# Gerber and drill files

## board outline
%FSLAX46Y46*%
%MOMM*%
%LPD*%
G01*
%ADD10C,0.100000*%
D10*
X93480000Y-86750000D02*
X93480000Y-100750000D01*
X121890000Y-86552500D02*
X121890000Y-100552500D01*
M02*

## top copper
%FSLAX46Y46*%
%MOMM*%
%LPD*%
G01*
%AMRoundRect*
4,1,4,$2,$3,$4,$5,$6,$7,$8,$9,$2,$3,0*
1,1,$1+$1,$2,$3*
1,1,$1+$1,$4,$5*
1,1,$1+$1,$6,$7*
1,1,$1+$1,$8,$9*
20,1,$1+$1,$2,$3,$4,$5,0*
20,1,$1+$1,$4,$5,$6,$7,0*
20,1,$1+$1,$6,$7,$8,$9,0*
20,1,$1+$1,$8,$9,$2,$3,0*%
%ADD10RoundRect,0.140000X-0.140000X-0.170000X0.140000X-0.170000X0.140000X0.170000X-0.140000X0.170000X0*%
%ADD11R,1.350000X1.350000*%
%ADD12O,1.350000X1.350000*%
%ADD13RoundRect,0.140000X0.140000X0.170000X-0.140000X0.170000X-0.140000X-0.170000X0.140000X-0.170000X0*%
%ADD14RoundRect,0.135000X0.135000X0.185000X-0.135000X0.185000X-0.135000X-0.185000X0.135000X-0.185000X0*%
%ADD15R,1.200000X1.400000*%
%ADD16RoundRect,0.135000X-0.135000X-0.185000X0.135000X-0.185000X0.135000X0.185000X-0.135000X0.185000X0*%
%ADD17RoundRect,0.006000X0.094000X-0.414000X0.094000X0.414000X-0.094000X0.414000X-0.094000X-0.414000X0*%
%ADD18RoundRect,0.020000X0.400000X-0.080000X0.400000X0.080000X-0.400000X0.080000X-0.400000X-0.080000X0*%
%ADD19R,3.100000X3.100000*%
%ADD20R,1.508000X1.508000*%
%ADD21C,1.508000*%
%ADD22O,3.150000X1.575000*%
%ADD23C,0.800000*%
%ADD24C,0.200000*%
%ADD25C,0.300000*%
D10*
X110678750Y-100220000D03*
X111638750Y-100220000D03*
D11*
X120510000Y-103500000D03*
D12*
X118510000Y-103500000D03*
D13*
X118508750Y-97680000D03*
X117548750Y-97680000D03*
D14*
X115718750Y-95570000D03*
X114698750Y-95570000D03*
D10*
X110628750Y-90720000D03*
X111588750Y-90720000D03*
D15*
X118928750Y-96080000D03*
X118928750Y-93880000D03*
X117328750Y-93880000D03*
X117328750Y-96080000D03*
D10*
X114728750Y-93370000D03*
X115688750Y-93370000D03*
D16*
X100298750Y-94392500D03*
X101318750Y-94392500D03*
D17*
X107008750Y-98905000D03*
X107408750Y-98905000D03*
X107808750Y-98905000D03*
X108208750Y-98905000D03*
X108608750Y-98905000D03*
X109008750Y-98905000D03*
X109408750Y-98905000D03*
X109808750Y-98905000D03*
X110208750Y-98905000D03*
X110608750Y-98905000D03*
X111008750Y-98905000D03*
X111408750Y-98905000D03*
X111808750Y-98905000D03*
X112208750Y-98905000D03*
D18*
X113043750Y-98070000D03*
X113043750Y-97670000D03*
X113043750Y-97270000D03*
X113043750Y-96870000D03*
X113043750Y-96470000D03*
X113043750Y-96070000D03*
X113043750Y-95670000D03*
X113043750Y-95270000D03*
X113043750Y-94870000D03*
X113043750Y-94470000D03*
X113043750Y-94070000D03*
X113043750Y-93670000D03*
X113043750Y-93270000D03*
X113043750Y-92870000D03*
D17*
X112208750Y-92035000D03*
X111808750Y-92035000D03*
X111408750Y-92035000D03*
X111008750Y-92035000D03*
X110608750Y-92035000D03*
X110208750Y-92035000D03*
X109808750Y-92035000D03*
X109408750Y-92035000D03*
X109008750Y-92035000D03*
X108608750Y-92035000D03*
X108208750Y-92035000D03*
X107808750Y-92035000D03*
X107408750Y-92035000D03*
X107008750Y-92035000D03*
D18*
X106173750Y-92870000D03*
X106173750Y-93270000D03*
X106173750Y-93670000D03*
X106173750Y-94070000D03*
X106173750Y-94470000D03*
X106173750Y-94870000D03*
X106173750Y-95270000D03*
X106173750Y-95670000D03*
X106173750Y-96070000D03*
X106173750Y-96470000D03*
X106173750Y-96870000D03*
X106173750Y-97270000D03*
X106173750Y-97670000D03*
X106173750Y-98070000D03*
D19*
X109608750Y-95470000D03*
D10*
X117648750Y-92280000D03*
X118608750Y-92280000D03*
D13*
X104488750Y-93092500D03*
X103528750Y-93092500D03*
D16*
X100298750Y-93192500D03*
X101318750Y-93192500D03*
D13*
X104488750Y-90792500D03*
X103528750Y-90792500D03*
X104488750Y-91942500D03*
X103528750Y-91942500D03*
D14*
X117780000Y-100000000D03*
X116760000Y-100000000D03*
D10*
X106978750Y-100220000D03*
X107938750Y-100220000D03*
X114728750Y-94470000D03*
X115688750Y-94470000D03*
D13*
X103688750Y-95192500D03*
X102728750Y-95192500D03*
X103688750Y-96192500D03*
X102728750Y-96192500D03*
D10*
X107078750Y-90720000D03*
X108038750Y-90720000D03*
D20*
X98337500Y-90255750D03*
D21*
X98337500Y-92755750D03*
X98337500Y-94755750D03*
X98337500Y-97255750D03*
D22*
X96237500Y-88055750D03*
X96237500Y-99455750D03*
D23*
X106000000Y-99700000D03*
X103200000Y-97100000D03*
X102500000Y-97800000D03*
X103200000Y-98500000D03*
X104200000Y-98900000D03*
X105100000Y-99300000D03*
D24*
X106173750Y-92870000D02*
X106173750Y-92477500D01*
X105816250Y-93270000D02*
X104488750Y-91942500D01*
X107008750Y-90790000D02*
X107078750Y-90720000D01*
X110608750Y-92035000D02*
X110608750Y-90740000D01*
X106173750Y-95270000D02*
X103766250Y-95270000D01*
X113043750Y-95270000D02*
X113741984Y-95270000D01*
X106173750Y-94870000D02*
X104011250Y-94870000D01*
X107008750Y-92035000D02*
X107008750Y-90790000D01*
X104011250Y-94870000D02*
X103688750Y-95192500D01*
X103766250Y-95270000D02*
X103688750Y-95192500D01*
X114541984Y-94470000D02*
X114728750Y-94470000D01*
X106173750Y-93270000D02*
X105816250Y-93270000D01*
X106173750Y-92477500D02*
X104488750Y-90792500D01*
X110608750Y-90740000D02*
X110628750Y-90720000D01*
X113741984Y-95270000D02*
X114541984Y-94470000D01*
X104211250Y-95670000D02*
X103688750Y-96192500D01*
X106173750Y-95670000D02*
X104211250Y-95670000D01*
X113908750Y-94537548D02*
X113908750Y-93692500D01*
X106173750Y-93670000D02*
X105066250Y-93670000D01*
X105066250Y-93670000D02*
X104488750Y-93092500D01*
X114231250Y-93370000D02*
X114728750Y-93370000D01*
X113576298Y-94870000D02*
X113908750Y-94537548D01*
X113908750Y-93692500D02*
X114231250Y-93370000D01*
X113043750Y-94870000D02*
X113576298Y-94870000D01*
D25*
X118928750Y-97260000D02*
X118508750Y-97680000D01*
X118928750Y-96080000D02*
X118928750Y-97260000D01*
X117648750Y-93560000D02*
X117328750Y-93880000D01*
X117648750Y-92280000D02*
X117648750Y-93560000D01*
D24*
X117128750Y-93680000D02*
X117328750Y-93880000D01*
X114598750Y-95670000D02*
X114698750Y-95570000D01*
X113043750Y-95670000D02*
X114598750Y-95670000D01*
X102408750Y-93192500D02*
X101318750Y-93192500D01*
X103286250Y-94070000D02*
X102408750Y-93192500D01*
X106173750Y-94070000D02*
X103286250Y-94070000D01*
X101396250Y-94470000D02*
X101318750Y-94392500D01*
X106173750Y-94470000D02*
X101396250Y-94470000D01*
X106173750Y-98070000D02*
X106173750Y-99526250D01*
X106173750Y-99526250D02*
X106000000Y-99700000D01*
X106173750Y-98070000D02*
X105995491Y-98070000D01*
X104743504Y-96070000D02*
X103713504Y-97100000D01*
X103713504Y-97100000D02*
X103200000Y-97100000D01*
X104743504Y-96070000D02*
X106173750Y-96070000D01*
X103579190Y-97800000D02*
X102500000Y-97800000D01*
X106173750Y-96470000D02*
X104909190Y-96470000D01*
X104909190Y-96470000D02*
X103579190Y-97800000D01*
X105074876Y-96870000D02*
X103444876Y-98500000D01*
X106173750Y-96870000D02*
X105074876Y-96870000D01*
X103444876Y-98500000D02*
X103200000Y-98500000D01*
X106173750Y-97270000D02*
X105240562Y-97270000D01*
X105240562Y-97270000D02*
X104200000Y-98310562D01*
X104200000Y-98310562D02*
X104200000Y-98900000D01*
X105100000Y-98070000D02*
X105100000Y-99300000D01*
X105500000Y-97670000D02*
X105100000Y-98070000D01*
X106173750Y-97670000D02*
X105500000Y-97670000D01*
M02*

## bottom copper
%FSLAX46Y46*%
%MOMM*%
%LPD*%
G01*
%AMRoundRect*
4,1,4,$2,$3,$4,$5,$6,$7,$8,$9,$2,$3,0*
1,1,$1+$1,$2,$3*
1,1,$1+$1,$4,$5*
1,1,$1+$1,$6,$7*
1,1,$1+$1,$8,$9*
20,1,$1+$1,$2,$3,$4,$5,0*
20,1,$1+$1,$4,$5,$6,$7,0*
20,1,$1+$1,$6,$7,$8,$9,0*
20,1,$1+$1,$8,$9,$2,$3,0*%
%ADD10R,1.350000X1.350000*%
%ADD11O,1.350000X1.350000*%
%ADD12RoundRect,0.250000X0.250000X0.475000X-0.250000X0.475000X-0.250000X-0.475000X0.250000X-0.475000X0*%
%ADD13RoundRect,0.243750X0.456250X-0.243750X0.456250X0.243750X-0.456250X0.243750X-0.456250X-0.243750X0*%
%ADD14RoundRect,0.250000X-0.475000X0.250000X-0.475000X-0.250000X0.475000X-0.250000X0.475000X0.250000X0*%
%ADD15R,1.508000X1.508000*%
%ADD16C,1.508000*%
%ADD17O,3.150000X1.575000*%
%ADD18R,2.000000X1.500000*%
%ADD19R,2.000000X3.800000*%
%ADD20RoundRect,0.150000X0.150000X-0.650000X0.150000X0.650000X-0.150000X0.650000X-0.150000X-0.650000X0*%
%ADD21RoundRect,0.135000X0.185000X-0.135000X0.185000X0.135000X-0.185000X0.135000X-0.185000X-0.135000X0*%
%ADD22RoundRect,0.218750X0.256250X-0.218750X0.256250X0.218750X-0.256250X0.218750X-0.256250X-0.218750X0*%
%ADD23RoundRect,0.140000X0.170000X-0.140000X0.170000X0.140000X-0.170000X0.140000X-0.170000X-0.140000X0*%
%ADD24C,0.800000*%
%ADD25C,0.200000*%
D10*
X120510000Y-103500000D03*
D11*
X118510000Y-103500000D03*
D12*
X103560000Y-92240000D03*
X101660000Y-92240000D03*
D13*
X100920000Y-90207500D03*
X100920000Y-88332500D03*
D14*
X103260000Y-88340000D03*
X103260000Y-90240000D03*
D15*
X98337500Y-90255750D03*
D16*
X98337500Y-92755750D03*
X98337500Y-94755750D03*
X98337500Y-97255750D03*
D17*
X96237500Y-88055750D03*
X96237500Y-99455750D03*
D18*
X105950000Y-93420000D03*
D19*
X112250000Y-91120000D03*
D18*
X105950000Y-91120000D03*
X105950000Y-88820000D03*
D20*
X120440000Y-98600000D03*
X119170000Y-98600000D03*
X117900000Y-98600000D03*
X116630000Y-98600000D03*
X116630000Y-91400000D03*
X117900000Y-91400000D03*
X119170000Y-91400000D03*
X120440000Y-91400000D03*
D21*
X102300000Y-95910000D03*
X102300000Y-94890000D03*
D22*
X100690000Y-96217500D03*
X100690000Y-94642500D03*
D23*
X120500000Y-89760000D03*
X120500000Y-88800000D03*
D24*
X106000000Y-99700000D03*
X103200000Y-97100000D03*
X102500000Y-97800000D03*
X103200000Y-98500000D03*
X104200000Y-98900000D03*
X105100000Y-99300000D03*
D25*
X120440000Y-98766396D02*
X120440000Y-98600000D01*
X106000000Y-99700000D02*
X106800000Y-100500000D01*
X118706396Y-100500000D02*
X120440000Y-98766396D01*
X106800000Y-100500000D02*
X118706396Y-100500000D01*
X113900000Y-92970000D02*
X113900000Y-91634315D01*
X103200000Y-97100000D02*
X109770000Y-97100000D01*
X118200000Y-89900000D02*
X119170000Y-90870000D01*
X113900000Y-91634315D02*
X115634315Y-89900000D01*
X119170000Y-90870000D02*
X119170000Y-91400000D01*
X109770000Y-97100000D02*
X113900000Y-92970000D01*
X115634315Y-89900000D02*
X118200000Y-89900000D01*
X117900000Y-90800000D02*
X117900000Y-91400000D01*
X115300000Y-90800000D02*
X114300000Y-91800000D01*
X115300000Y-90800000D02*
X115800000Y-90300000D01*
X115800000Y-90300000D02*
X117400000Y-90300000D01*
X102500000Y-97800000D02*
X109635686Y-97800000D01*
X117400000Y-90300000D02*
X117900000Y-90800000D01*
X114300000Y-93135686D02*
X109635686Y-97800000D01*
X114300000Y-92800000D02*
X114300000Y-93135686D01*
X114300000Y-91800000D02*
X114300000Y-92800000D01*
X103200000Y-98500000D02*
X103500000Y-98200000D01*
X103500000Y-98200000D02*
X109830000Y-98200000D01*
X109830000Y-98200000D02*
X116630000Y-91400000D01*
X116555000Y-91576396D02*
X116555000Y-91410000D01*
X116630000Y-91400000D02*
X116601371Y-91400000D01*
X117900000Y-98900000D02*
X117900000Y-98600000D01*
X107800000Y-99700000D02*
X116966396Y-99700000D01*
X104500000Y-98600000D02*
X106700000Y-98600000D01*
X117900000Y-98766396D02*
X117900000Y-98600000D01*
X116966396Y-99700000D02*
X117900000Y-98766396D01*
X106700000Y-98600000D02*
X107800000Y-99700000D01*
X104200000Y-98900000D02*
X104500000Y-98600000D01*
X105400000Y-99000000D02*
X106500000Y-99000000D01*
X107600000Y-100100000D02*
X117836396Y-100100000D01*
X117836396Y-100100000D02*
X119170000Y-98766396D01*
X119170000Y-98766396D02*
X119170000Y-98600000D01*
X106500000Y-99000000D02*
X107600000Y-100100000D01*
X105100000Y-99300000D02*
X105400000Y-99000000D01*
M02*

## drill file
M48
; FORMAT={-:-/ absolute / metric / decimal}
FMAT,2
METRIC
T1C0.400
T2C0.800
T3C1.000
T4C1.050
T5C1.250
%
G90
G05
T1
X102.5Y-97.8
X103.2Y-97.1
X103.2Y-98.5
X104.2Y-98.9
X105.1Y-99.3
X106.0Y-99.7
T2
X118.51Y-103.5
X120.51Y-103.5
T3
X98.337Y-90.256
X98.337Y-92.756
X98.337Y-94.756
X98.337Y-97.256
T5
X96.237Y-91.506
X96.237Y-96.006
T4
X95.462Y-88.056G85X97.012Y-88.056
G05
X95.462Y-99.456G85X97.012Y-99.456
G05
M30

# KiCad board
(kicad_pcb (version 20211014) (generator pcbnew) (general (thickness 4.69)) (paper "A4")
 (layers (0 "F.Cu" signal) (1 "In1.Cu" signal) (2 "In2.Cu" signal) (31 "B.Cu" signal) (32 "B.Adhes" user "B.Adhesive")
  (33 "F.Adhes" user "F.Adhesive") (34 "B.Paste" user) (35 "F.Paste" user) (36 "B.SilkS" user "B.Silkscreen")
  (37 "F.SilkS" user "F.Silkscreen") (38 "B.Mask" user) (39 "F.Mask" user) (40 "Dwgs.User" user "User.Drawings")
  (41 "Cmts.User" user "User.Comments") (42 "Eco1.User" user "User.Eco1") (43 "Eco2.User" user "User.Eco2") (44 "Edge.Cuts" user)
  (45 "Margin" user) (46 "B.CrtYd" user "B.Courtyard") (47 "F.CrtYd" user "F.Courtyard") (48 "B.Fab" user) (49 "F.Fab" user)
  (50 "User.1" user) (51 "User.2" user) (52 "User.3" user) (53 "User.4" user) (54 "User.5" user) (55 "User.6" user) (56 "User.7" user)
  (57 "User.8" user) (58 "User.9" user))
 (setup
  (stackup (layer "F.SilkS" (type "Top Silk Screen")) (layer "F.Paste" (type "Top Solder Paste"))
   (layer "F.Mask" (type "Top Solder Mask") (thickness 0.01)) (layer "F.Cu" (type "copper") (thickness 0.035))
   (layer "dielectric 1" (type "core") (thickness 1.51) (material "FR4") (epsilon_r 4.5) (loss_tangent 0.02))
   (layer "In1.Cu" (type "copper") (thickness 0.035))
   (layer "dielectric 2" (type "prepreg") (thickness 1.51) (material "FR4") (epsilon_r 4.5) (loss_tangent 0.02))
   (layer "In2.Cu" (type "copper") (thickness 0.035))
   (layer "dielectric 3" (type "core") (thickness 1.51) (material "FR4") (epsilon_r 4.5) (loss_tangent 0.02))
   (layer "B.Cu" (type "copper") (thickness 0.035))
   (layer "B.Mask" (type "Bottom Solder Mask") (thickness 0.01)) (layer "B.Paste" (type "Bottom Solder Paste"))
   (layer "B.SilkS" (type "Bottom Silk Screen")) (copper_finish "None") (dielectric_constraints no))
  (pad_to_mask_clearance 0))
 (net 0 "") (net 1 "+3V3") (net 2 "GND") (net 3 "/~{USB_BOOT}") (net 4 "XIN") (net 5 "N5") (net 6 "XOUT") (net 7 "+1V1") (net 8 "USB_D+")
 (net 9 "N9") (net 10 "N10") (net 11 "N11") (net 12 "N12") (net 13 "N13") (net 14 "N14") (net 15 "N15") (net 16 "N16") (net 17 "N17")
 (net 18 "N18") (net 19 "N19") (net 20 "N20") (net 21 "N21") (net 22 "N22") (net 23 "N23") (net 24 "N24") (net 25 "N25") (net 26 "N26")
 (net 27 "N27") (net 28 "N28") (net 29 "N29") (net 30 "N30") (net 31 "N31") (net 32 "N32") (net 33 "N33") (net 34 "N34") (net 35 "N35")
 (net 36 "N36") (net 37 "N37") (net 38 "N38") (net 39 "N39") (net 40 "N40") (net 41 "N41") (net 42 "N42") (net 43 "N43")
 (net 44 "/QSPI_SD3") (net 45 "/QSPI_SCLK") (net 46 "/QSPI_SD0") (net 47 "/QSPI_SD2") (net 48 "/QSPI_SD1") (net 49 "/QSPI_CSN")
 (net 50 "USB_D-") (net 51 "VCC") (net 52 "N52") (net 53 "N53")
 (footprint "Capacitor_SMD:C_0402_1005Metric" (layer "F.Cu") (at 111.15875 100.22)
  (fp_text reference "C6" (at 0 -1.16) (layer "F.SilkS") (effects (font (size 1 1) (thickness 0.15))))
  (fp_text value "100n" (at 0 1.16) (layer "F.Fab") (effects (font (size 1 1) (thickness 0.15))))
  (pad "1" smd roundrect (at -0.48 0) (size 0.56 0.62) (layers "F.Cu" "F.Paste" "F.Mask") (roundrect_rratio 0.25) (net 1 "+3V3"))
  (pad "2" smd roundrect (at 0.48 0) (size 0.56 0.62) (layers "F.Cu" "F.Paste" "F.Mask") (roundrect_rratio 0.25) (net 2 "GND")))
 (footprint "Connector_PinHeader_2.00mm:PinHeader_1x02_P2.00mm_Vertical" (layer "F.Cu") (at 120.51 103.5 -90)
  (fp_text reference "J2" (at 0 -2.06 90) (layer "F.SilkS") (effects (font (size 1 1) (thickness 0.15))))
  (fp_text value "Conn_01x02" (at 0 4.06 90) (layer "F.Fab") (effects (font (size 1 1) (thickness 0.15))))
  (pad "1" thru_hole rect (at 0 0 270) (size 1.35 1.35) (drill 0.8) (layers *.Cu *.Mask) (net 2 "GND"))
  (pad "2" thru_hole oval (at 0 2 270) (size 1.35 1.35) (drill 0.8) (layers *.Cu *.Mask) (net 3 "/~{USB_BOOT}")))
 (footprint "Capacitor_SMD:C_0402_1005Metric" (layer "F.Cu") (at 118.02875 97.68 180)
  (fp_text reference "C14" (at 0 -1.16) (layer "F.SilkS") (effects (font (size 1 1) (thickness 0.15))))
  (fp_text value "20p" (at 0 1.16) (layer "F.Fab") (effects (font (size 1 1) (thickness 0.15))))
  (pad "1" smd roundrect (at -0.48 0 180) (size 0.56 0.62) (layers "F.Cu" "F.Paste" "F.Mask") (roundrect_rratio 0.25) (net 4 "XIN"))
  (pad "2" smd roundrect (at 0.48 0 180) (size 0.56 0.62) (layers "F.Cu" "F.Paste" "F.Mask") (roundrect_rratio 0.25) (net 2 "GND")))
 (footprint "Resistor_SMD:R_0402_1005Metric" (layer "F.Cu") (at 115.20875 95.57 180)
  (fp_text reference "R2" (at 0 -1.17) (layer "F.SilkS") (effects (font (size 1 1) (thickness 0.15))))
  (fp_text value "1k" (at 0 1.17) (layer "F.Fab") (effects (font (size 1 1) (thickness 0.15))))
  (pad "1" smd roundrect (at -0.51 0 180) (size 0.54 0.64) (layers "F.Cu" "F.Paste" "F.Mask") (roundrect_rratio 0.25) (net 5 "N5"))
  (pad "2" smd roundrect (at 0.51 0 180) (size 0.54 0.64) (layers "F.Cu" "F.Paste" "F.Mask") (roundrect_rratio 0.25) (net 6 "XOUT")))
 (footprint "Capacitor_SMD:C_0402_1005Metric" (layer "F.Cu") (at 111.10875 90.72)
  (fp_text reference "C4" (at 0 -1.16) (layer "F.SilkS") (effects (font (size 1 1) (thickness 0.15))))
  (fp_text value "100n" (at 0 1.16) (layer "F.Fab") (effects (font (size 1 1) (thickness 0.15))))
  (pad "1" smd roundrect (at -0.48 0) (size 0.56 0.62) (layers "F.Cu" "F.Paste" "F.Mask") (roundrect_rratio 0.25) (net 1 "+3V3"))
  (pad "2" smd roundrect (at 0.48 0) (size 0.56 0.62) (layers "F.Cu" "F.Paste" "F.Mask") (roundrect_rratio 0.25) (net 2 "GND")))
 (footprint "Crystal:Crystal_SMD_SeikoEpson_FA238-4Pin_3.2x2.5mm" (layer "F.Cu") (at 118.12875 94.98 90)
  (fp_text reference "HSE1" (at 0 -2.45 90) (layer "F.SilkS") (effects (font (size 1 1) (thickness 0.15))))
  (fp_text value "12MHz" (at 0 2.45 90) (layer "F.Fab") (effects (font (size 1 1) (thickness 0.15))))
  (pad "1" smd rect (at -1.1 0.8 90) (size 1.4 1.2) (layers "F.Cu" "F.Paste" "F.Mask") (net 4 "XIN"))
  (pad "2" smd rect (at 1.1 0.8 90) (size 1.4 1.2) (layers "F.Cu" "F.Paste" "F.Mask") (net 2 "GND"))
  (pad "3" smd rect (at 1.1 -0.8 90) (size 1.4 1.2) (layers "F.Cu" "F.Paste" "F.Mask") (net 5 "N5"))
  (pad "4" smd rect (at -1.1 -0.8 90) (size 1.4 1.2) (layers "F.Cu" "F.Paste" "F.Mask") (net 2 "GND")))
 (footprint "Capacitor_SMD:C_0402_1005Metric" (layer "F.Cu") (at 115.20875 93.37)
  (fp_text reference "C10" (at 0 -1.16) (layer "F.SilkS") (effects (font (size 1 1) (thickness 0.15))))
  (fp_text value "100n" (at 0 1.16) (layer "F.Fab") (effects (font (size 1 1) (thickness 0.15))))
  (pad "1" smd roundrect (at -0.48 0) (size 0.56 0.62) (layers "F.Cu" "F.Paste" "F.Mask") (roundrect_rratio 0.25) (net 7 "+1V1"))
  (pad "2" smd roundrect (at 0.48 0) (size 0.56 0.62) (layers "F.Cu" "F.Paste" "F.Mask") (roundrect_rratio 0.25) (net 2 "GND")))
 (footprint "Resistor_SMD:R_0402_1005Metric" (layer "F.Cu") (at 100.80875 94.3925)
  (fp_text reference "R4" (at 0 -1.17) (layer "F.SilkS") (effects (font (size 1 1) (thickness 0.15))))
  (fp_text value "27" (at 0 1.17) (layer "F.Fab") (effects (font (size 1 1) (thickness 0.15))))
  (pad "1" smd roundrect (at -0.51 0) (size 0.54 0.64) (layers "F.Cu" "F.Paste" "F.Mask") (roundrect_rratio 0.25) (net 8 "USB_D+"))
  (pad "2" smd roundrect (at 0.51 0) (size 0.54 0.64) (layers "F.Cu" "F.Paste" "F.Mask") (roundrect_rratio 0.25) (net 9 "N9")))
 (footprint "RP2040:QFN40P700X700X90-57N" (layer "F.Cu") (at 109.60875 95.47 90)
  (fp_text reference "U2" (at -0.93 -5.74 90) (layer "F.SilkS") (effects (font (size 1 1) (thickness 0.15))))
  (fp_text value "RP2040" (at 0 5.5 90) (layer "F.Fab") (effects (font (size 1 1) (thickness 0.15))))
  (pad "1" smd roundrect locked (at -3.435 -2.6 90) (size 0.84 0.2) (layers "F.Cu" "F.Paste" "F.Mask") (roundrect_rratio 0.03)
   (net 1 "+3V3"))
  (pad "2" smd roundrect locked (at -3.435 -2.2 90) (size 0.84 0.2) (layers "F.Cu" "F.Paste" "F.Mask") (roundrect_rratio 0.03)
   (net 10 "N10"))
  (pad "3" smd roundrect locked (at -3.435 -1.8 90) (size 0.84 0.2) (layers "F.Cu" "F.Paste" "F.Mask") (roundrect_rratio 0.03)
   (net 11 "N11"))
  (pad "4" smd roundrect locked (at -3.435 -1.4 90) (size 0.84 0.2) (layers "F.Cu" "F.Paste" "F.Mask") (roundrect_rratio 0.03)
   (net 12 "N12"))
  (pad "5" smd roundrect locked (at -3.435 -1 90) (size 0.84 0.2) (layers "F.Cu" "F.Paste" "F.Mask") (roundrect_rratio 0.03) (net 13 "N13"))
  (pad "6" smd roundrect locked (at -3.435 -0.6 90) (size 0.84 0.2) (layers "F.Cu" "F.Paste" "F.Mask") (roundrect_rratio 0.03)
   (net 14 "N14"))
  (pad "7" smd roundrect locked (at -3.435 -0.2 90) (size 0.84 0.2) (layers "F.Cu" "F.Paste" "F.Mask") (roundrect_rratio 0.03)
   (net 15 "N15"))
  (pad "8" smd roundrect locked (at -3.435 0.2 90) (size 0.84 0.2) (layers "F.Cu" "F.Paste" "F.Mask") (roundrect_rratio 0.03) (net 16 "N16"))
  (pad "9" smd roundrect locked (at -3.435 0.6 90) (size 0.84 0.2) (layers "F.Cu" "F.Paste" "F.Mask") (roundrect_rratio 0.03) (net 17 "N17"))
  (pad "10" smd roundrect locked (at -3.435 1 90) (size 0.84 0.2) (layers "F.Cu" "F.Paste" "F.Mask") (roundrect_rratio 0.03) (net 1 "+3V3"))
  (pad "11" smd roundrect locked (at -3.435 1.4 90) (size 0.84 0.2) (layers "F.Cu" "F.Paste" "F.Mask") (roundrect_rratio 0.03)
   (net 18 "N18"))
  (pad "12" smd roundrect locked (at -3.435 1.8 90) (size 0.84 0.2) (layers "F.Cu" "F.Paste" "F.Mask") (roundrect_rratio 0.03)
   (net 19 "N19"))
  (pad "13" smd roundrect locked (at -3.435 2.2 90) (size 0.84 0.2) (layers "F.Cu" "F.Paste" "F.Mask") (roundrect_rratio 0.03)
   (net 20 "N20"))
  (pad "14" smd roundrect locked (at -3.435 2.6 90) (size 0.84 0.2) (layers "F.Cu" "F.Paste" "F.Mask") (roundrect_rratio 0.03)
   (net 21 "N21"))
  (pad "15" smd roundrect locked (at -2.6 3.435 90) (size 0.2 0.84) (layers "F.Cu" "F.Paste" "F.Mask") (roundrect_rratio 0.1) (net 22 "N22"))
  (pad "16" smd roundrect locked (at -2.2 3.435 90) (size 0.2 0.84) (layers "F.Cu" "F.Paste" "F.Mask") (roundrect_rratio 0.1) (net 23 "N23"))
  (pad "17" smd roundrect locked (at -1.8 3.435 90) (size 0.2 0.84) (layers "F.Cu" "F.Paste" "F.Mask") (roundrect_rratio 0.1) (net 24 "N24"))
  (pad "18" smd roundrect locked (at -1.4 3.435 90) (size 0.2 0.84) (layers "F.Cu" "F.Paste" "F.Mask") (roundrect_rratio 0.1) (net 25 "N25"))
  (pad "19" smd roundrect locked (at -1 3.435 90) (size 0.2 0.84) (layers "F.Cu" "F.Paste" "F.Mask") (roundrect_rratio 0.1) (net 2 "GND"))
  (pad "20" smd roundrect locked (at -0.6 3.435 90) (size 0.2 0.84) (layers "F.Cu" "F.Paste" "F.Mask") (roundrect_rratio 0.1) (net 4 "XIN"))
  (pad "21" smd roundrect locked (at -0.2 3.435 90) (size 0.2 0.84) (layers "F.Cu" "F.Paste" "F.Mask") (roundrect_rratio 0.1) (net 6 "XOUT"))
  (pad "22" smd roundrect locked (at 0.2 3.435 90) (size 0.2 0.84) (layers "F.Cu" "F.Paste" "F.Mask") (roundrect_rratio 0.1) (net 1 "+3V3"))
  (pad "23" smd roundrect locked (at 0.6 3.435 90) (size 0.2 0.84) (layers "F.Cu" "F.Paste" "F.Mask") (roundrect_rratio 0.1) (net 7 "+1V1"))
  (pad "24" smd roundrect locked (at 1 3.435 90) (size 0.2 0.84) (layers "F.Cu" "F.Paste" "F.Mask") (roundrect_rratio 0.1) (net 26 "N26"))
  (pad "25" smd roundrect locked (at 1.4 3.435 90) (size 0.2 0.84) (layers "F.Cu" "F.Paste" "F.Mask") (roundrect_rratio 0.1) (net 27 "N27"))
  (pad "26" smd roundrect locked (at 1.8 3.435 90) (size 0.2 0.84) (layers "F.Cu" "F.Paste" "F.Mask") (roundrect_rratio 0.1) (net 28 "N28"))
  (pad "27" smd roundrect locked (at 2.2 3.435 90) (size 0.2 0.84) (layers "F.Cu" "F.Paste" "F.Mask") (roundrect_rratio 0.1) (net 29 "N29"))
  (pad "28" smd roundrect locked (at 2.6 3.435 90) (size 0.2 0.84) (layers "F.Cu" "F.Paste" "F.Mask") (roundrect_rratio 0.1) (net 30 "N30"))
  (pad "29" smd roundrect locked (at 3.435 2.6 90) (size 0.84 0.2) (layers "F.Cu" "F.Paste" "F.Mask") (roundrect_rratio 0.03) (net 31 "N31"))
  (pad "30" smd roundrect locked (at 3.435 2.2 90) (size 0.84 0.2) (layers "F.Cu" "F.Paste" "F.Mask") (roundrect_rratio 0.03) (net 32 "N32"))
  (pad "31" smd roundrect locked (at 3.435 1.8 90) (size 0.84 0.2) (layers "F.Cu" "F.Paste" "F.Mask") (roundrect_rratio 0.03) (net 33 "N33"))
  (pad "32" smd roundrect locked (at 3.435 1.4 90) (size 0.84 0.2) (layers "F.Cu" "F.Paste" "F.Mask") (roundrect_rratio 0.03) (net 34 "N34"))
  (pad "33" smd roundrect locked (at 3.435 1 90) (size 0.84 0.2) (layers "F.Cu" "F.Paste" "F.Mask") (roundrect_rratio 0.03) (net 1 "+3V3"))
  (pad "34" smd roundrect locked (at 3.435 0.6 90) (size 0.84 0.2) (layers "F.Cu" "F.Paste" "F.Mask") (roundrect_rratio 0.03) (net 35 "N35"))
  (pad "35" smd roundrect locked (at 3.435 0.2 90) (size 0.84 0.2) (layers "F.Cu" "F.Paste" "F.Mask") (roundrect_rratio 0.03) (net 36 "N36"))
  (pad "36" smd roundrect locked (at 3.435 -0.2 90) (size 0.84 0.2) (layers "F.Cu" "F.Paste" "F.Mask") (roundrect_rratio 0.03)
   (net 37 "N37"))
  (pad "37" smd roundrect locked (at 3.435 -0.6 90) (size 0.84 0.2) (layers "F.Cu" "F.Paste" "F.Mask") (roundrect_rratio 0.03)
   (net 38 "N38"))
  (pad "38" smd roundrect locked (at 3.435 -1 90) (size 0.84 0.2) (layers "F.Cu" "F.Paste" "F.Mask") (roundrect_rratio 0.03) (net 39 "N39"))
  (pad "39" smd roundrect locked (at 3.435 -1.4 90) (size 0.84 0.2) (layers "F.Cu" "F.Paste" "F.Mask") (roundrect_rratio 0.03)
   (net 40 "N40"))
  (pad "40" smd roundrect locked (at 3.435 -1.8 90) (size 0.84 0.2) (layers "F.Cu" "F.Paste" "F.Mask") (roundrect_rratio 0.03)
   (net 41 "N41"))
  (pad "41" smd roundrect locked (at 3.435 -2.2 90) (size 0.84 0.2) (layers "F.Cu" "F.Paste" "F.Mask") (roundrect_rratio 0.03)
   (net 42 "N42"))
  (pad "42" smd roundrect locked (at 3.435 -2.6 90) (size 0.84 0.2) (layers "F.Cu" "F.Paste" "F.Mask") (roundrect_rratio 0.03)
   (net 1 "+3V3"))
  (pad "43" smd roundrect locked (at 2.6 -3.435 90) (size 0.2 0.84) (layers "F.Cu" "F.Paste" "F.Mask") (roundrect_rratio 0.1) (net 1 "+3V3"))
  (pad "44" smd roundrect locked (at 2.2 -3.435 90) (size 0.2 0.84) (layers "F.Cu" "F.Paste" "F.Mask") (roundrect_rratio 0.1) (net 1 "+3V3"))
  (pad "45" smd roundrect locked (at 1.8 -3.435 90) (size 0.2 0.84) (layers "F.Cu" "F.Paste" "F.Mask") (roundrect_rratio 0.1) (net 7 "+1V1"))
  (pad "46" smd roundrect locked (at 1.4 -3.435 90) (size 0.2 0.84) (layers "F.Cu" "F.Paste" "F.Mask") (roundrect_rratio 0.1) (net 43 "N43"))
  (pad "47" smd roundrect locked (at 1 -3.435 90) (size 0.2 0.84) (layers "F.Cu" "F.Paste" "F.Mask") (roundrect_rratio 0.1) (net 9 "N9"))
  (pad "48" smd roundrect locked (at 0.6 -3.435 90) (size 0.2 0.84) (layers "F.Cu" "F.Paste" "F.Mask") (roundrect_rratio 0.1) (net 1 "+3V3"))
  (pad "49" smd roundrect locked (at 0.2 -3.435 90) (size 0.2 0.84) (layers "F.Cu" "F.Paste" "F.Mask") (roundrect_rratio 0.1) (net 1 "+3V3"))
  (pad "50" smd roundrect locked (at -0.2 -3.435 90) (size 0.2 0.84) (layers "F.Cu" "F.Paste" "F.Mask") (roundrect_rratio 0.1)
   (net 7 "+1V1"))
  (pad "51" smd roundrect locked (at -0.6 -3.435 90) (size 0.2 0.84) (layers "F.Cu" "F.Paste" "F.Mask") (roundrect_rratio 0.1)
   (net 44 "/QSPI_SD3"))
  (pad "52" smd roundrect locked (at -1 -3.435 90) (size 0.2 0.84) (layers "F.Cu" "F.Paste" "F.Mask") (roundrect_rratio 0.1)
   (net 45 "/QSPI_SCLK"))
  (pad "53" smd roundrect locked (at -1.4 -3.435 90) (size 0.2 0.84) (layers "F.Cu" "F.Paste" "F.Mask") (roundrect_rratio 0.1)
   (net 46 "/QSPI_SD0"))
  (pad "54" smd roundrect locked (at -1.8 -3.435 90) (size 0.2 0.84) (layers "F.Cu" "F.Paste" "F.Mask") (roundrect_rratio 0.1)
   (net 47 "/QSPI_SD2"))
  (pad "55" smd roundrect locked (at -2.2 -3.435 90) (size 0.2 0.84) (layers "F.Cu" "F.Paste" "F.Mask") (roundrect_rratio 0.1)
   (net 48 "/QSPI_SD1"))
  (pad "56" smd roundrect locked (at -2.6 -3.435 90) (size 0.2 0.84) (layers "F.Cu" "F.Paste" "F.Mask") (roundrect_rratio 0.1)
   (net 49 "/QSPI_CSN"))
  (pad "57" smd rect locked (at 0 0 90) (size 3.1 3.1) (layers "F.Cu" "F.Mask") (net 2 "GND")))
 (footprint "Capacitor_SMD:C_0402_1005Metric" (layer "F.Cu") (at 118.12875 92.28)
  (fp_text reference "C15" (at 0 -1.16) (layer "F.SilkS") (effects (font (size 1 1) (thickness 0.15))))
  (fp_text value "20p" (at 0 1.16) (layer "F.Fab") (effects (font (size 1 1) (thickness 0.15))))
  (pad "1" smd roundrect (at -0.48 0) (size 0.56 0.62) (layers "F.Cu" "F.Paste" "F.Mask") (roundrect_rratio 0.25) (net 5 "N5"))
  (pad "2" smd roundrect (at 0.48 0) (size 0.56 0.62) (layers "F.Cu" "F.Paste" "F.Mask") (roundrect_rratio 0.25) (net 2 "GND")))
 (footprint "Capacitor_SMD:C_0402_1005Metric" (layer "F.Cu") (at 104.00875 93.0925 180)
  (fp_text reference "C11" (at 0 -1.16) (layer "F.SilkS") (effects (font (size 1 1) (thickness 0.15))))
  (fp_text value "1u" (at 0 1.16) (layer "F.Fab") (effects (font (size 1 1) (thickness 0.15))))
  (pad "1" smd roundrect (at -0.48 0 180) (size 0.56 0.62) (layers "F.Cu" "F.Paste" "F.Mask") (roundrect_rratio 0.25) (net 7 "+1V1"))
  (pad "2" smd roundrect (at 0.48 0 180) (size 0.56 0.62) (layers "F.Cu" "F.Paste" "F.Mask") (roundrect_rratio 0.25) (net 2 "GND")))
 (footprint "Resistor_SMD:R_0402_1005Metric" (layer "F.Cu") (at 100.80875 93.1925)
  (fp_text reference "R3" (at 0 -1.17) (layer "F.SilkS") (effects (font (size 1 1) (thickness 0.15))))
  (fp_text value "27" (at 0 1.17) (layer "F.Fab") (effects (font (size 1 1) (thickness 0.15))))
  (pad "1" smd roundrect (at -0.51 0) (size 0.54 0.64) (layers "F.Cu" "F.Paste" "F.Mask") (roundrect_rratio 0.25) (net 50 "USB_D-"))
  (pad "2" smd roundrect (at 0.51 0) (size 0.54 0.64) (layers "F.Cu" "F.Paste" "F.Mask") (roundrect_rratio 0.25) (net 43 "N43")))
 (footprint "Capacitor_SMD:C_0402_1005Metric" (layer "F.Cu") (at 104.00875 90.7925 180)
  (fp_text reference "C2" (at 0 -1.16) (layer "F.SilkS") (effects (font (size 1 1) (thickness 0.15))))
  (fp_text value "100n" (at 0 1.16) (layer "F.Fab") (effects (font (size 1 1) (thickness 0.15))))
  (pad "1" smd roundrect (at -0.48 0 180) (size 0.56 0.62) (layers "F.Cu" "F.Paste" "F.Mask") (roundrect_rratio 0.25) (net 1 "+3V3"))
  (pad "2" smd roundrect (at 0.48 0 180) (size 0.56 0.62) (layers "F.Cu" "F.Paste" "F.Mask") (roundrect_rratio 0.25) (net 2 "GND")))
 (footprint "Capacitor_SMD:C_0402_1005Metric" (layer "F.Cu") (at 104.00875 91.9425 180)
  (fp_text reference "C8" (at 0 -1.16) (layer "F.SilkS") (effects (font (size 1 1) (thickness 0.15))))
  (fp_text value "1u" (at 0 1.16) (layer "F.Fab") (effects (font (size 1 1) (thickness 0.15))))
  (pad "1" smd roundrect (at -0.48 0 180) (size 0.56 0.62) (layers "F.Cu" "F.Paste" "F.Mask") (roundrect_rratio 0.25) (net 1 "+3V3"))
  (pad "2" smd roundrect (at 0.48 0 180) (size 0.56 0.62) (layers "F.Cu" "F.Paste" "F.Mask") (roundrect_rratio 0.25) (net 2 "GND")))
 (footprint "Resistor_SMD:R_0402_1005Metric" (layer "F.Cu") (at 117.27 100 180)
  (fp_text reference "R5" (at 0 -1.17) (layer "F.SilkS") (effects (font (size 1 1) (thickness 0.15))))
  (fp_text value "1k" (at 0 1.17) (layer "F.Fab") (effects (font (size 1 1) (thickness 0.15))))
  (pad "1" smd roundrect (at -0.51 0 180) (size 0.54 0.64) (layers "F.Cu" "F.Paste" "F.Mask") (roundrect_rratio 0.25) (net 3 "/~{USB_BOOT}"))
  (pad "2" smd roundrect (at 0.51 0 180) (size 0.54 0.64) (layers "F.Cu" "F.Paste" "F.Mask") (roundrect_rratio 0.25) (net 49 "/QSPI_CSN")))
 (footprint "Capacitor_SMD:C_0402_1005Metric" (layer "F.Cu") (at 107.45875 100.22)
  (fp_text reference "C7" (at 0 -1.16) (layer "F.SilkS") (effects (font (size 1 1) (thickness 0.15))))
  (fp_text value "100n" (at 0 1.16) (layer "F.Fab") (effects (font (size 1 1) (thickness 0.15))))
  (pad "1" smd roundrect (at -0.48 0) (size 0.56 0.62) (layers "F.Cu" "F.Paste" "F.Mask") (roundrect_rratio 0.25) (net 1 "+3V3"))
  (pad "2" smd roundrect (at 0.48 0) (size 0.56 0.62) (layers "F.Cu" "F.Paste" "F.Mask") (roundrect_rratio 0.25) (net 2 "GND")))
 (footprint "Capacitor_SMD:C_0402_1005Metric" (layer "F.Cu") (at 115.20875 94.47)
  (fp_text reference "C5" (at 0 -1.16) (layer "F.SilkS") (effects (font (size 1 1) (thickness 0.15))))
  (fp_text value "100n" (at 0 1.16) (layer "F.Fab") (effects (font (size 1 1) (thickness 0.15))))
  (pad "1" smd roundrect (at -0.48 0) (size 0.56 0.62) (layers "F.Cu" "F.Paste" "F.Mask") (roundrect_rratio 0.25) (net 1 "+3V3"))
  (pad "2" smd roundrect (at 0.48 0) (size 0.56 0.62) (layers "F.Cu" "F.Paste" "F.Mask") (roundrect_rratio 0.25) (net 2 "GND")))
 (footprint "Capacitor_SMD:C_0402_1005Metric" (layer "F.Cu") (at 103.20875 95.1925 180)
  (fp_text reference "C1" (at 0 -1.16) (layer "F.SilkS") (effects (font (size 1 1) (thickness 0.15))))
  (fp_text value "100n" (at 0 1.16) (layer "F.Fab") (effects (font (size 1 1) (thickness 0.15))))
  (pad "1" smd roundrect (at -0.48 0 180) (size 0.56 0.62) (layers "F.Cu" "F.Paste" "F.Mask") (roundrect_rratio 0.25) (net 1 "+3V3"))
  (pad "2" smd roundrect (at 0.48 0 180) (size 0.56 0.62) (layers "F.Cu" "F.Paste" "F.Mask") (roundrect_rratio 0.25) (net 2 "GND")))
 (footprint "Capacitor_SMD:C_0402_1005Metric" (layer "F.Cu") (at 103.20875 96.1925 180)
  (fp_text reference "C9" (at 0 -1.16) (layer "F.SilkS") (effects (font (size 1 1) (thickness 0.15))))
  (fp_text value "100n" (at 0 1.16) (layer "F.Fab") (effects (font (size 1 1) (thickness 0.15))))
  (pad "1" smd roundrect (at -0.48 0 180) (size 0.56 0.62) (layers "F.Cu" "F.Paste" "F.Mask") (roundrect_rratio 0.25) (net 7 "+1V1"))
  (pad "2" smd roundrect (at 0.48 0 180) (size 0.56 0.62) (layers "F.Cu" "F.Paste" "F.Mask") (roundrect_rratio 0.25) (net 2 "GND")))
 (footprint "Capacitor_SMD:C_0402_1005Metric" (layer "F.Cu") (at 107.55875 90.72)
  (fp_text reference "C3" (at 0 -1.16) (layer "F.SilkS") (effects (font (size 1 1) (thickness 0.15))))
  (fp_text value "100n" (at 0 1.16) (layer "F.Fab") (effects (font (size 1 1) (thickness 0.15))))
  (pad "1" smd roundrect (at -0.48 0) (size 0.56 0.62) (layers "F.Cu" "F.Paste" "F.Mask") (roundrect_rratio 0.25) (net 1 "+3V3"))
  (pad "2" smd roundrect (at 0.48 0) (size 0.56 0.62) (layers "F.Cu" "F.Paste" "F.Mask") (roundrect_rratio 0.25) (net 2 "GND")))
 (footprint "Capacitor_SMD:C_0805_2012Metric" (layer "B.Cu") (at 102.61 92.24 180)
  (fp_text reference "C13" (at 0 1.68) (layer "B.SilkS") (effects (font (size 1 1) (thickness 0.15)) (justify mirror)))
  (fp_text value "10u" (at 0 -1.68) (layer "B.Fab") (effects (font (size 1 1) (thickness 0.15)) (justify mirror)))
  (pad "1" smd roundrect (at -0.95 0 180) (size 1 1.45) (layers "B.Cu" "B.Paste" "B.Mask") (roundrect_rratio 0.25) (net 1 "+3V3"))
  (pad "2" smd roundrect (at 0.95 0 180) (size 1 1.45) (layers "B.Cu" "B.Paste" "B.Mask") (roundrect_rratio 0.25) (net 2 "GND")))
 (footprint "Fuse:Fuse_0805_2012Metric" (layer "B.Cu") (at 100.92 89.27 90)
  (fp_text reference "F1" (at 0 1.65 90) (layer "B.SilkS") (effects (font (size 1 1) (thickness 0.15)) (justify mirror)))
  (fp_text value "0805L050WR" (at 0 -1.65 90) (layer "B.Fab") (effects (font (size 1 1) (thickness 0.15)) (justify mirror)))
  (pad "1" smd roundrect (at -0.9375 0 90) (size 0.975 1.4) (layers "B.Cu" "B.Paste" "B.Mask") (roundrect_rratio 0.25) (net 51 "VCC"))
  (pad "2" smd roundrect (at 0.9375 0 90) (size 0.975 1.4) (layers "B.Cu" "B.Paste" "B.Mask") (roundrect_rratio 0.25) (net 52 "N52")))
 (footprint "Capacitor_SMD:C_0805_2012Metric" (layer "B.Cu") (at 103.26 89.29 -90)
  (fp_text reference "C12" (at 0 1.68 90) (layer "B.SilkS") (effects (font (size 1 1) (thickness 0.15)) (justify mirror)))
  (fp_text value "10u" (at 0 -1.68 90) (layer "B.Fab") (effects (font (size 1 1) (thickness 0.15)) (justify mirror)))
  (pad "1" smd roundrect (at -0.95 0 270) (size 1 1.45) (layers "B.Cu" "B.Paste" "B.Mask") (roundrect_rratio 0.25) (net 52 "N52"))
  (pad "2" smd roundrect (at 0.95 0 270) (size 1 1.45) (layers "B.Cu" "B.Paste" "B.Mask") (roundrect_rratio 0.25) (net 2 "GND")))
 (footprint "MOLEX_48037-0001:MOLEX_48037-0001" (layer "B.Cu") (at 96.2375 93.75575 90)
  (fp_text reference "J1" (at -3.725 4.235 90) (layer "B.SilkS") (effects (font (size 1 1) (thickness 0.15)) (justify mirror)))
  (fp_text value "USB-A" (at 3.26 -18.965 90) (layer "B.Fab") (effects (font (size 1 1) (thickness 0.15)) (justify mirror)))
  (pad "" np_thru_hole circle locked (at -2.25 0 90) (size 1.25 1.25) (drill 1.25) (layers *.Cu *.Mask))
  (pad "" np_thru_hole circle locked (at 2.25 0 90) (size 1.25 1.25) (drill 1.25) (layers *.Cu *.Mask))
  (pad "1" thru_hole rect locked (at 3.5 2.1 90) (size 1.508 1.508) (drill 1) (layers *.Cu *.Mask) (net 51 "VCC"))
  (pad "2" thru_hole circle locked (at 1 2.1 90) (size 1.508 1.508) (drill 1) (layers *.Cu *.Mask) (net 50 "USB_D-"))
  (pad "3" thru_hole circle locked (at -1 2.1 90) (size 1.508 1.508) (drill 1) (layers *.Cu *.Mask) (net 8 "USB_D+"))
  (pad "4" thru_hole circle locked (at -3.5 2.1 90) (size 1.508 1.508) (drill 1) (layers *.Cu *.Mask) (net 2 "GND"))
  (pad "S1" thru_hole oval locked (at 5.7 0 90) (size 1.575 3.15) (drill oval 1.05 2.6) (layers *.Cu *.Mask) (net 2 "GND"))
  (pad "S2" thru_hole oval locked (at -5.7 0 90) (size 1.575 3.15) (drill oval 1.05 2.6) (layers *.Cu *.Mask) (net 2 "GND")))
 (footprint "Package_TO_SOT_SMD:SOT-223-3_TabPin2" (layer "B.Cu") (at 109.1 91.12)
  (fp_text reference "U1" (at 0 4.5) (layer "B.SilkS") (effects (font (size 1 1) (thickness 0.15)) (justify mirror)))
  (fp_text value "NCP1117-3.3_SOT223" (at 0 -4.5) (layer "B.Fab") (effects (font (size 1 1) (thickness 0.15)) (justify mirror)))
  (pad "1" smd rect (at -3.15 2.3) (size 2 1.5) (layers "B.Cu" "B.Paste" "B.Mask") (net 2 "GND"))
  (pad "2" smd rect (at 3.15 0) (size 2 3.8) (layers "B.Cu" "B.Paste" "B.Mask") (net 1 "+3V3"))
  (pad "2" smd rect (at -3.15 0) (size 2 1.5) (layers "B.Cu" "B.Paste" "B.Mask") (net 1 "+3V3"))
  (pad "3" smd rect (at -3.15 -2.3) (size 2 1.5) (layers "B.Cu" "B.Paste" "B.Mask") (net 52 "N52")))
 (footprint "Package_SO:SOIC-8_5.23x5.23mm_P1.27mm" (layer "B.Cu") (at 118.535 95 90)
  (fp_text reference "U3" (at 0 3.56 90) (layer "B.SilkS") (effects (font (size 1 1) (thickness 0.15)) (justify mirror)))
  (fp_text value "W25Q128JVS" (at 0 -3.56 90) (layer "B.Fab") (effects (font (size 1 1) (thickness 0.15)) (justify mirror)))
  (pad "1" smd roundrect (at -3.6 1.905 90) (size 1.6 0.6) (layers "B.Cu" "B.Paste" "B.Mask") (roundrect_rratio 0.25) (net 49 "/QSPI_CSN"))
  (pad "2" smd roundrect (at -3.6 0.635 90) (size 1.6 0.6) (layers "B.Cu" "B.Paste" "B.Mask") (roundrect_rratio 0.25) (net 48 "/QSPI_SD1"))
  (pad "3" smd roundrect (at -3.6 -0.635 90) (size 1.6 0.6) (layers "B.Cu" "B.Paste" "B.Mask") (roundrect_rratio 0.25) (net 47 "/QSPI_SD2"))
  (pad "4" smd roundrect (at -3.6 -1.905 90) (size 1.6 0.6) (layers "B.Cu" "B.Paste" "B.Mask") (roundrect_rratio 0.25) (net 2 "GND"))
  (pad "5" smd roundrect (at 3.6 -1.905 90) (size 1.6 0.6) (layers "B.Cu" "B.Paste" "B.Mask") (roundrect_rratio 0.25) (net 46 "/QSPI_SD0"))
  (pad "6" smd roundrect (at 3.6 -0.635 90) (size 1.6 0.6) (layers "B.Cu" "B.Paste" "B.Mask") (roundrect_rratio 0.25) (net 45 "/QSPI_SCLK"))
  (pad "7" smd roundrect (at 3.6 0.635 90) (size 1.6 0.6) (layers "B.Cu" "B.Paste" "B.Mask") (roundrect_rratio 0.25) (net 44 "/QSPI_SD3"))
  (pad "8" smd roundrect (at 3.6 1.905 90) (size 1.6 0.6) (layers "B.Cu" "B.Paste" "B.Mask") (roundrect_rratio 0.25) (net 1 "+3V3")))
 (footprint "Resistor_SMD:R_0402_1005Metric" (layer "B.Cu") (at 102.3 95.4 90)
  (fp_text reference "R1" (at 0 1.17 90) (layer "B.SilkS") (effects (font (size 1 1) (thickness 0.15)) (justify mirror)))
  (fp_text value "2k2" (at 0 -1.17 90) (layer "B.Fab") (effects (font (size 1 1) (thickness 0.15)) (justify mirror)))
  (pad "1" smd roundrect (at -0.51 0 90) (size 0.54 0.64) (layers "B.Cu" "B.Paste" "B.Mask") (roundrect_rratio 0.25) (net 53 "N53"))
  (pad "2" smd roundrect (at 0.51 0 90) (size 0.54 0.64) (layers "B.Cu" "B.Paste" "B.Mask") (roundrect_rratio 0.25) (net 2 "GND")))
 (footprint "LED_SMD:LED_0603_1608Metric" (layer "B.Cu") (at 100.69 95.43 90)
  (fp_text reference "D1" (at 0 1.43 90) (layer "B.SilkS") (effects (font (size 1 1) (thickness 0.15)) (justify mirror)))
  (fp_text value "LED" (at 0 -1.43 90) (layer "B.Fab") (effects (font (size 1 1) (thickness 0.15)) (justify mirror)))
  (pad "1" smd roundrect (at -0.7875 0 90) (size 0.875 0.95) (layers "B.Cu" "B.Paste" "B.Mask") (roundrect_rratio 0.25) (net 53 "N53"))
  (pad "2" smd roundrect (at 0.7875 0 90) (size 0.875 0.95) (layers "B.Cu" "B.Paste" "B.Mask") (roundrect_rratio 0.25) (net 1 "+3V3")))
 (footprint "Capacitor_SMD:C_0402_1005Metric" (layer "B.Cu") (at 120.5 89.28 90)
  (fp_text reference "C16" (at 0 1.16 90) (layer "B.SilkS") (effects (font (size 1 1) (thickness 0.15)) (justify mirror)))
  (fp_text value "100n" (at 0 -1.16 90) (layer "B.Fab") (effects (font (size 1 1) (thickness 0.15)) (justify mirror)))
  (pad "1" smd roundrect (at -0.48 0 90) (size 0.56 0.62) (layers "B.Cu" "B.Paste" "B.Mask") (roundrect_rratio 0.25) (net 1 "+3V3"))
  (pad "2" smd roundrect (at 0.48 0 90) (size 0.56 0.62) (layers "B.Cu" "B.Paste" "B.Mask") (roundrect_rratio 0.25) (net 2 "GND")))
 (gr_line (start 93.48 86.75) (end 93.48 100.75) (layer "Edge.Cuts") (width 0.1))
 (gr_line (start 121.89 86.5525) (end 121.89 100.5525) (layer "Edge.Cuts") (width 0.1))
 (segment (start 106.17375 92.87) (end 106.17375 92.4775) (width 0.2) (layer "F.Cu") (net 1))
 (segment (start 105.81625 93.27) (end 104.48875 91.9425) (width 0.2) (layer "F.Cu") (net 1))
 (segment (start 107.00875 90.79) (end 107.07875 90.72) (width 0.2) (layer "F.Cu") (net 1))
 (segment (start 110.60875 92.035) (end 110.60875 90.74) (width 0.2) (layer "F.Cu") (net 1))
 (segment (start 106.17375 95.27) (end 103.76625 95.27) (width 0.2) (layer "F.Cu") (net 1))
 (segment (start 113.04375 95.27) (end 113.741984 95.27) (width 0.2) (layer "F.Cu") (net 1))
 (segment (start 106.17375 94.87) (end 104.01125 94.87) (width 0.2) (layer "F.Cu") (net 1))
 (segment (start 107.00875 92.035) (end 107.00875 90.79) (width 0.2) (layer "F.Cu") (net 1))
 (segment (start 104.01125 94.87) (end 103.68875 95.1925) (width 0.2) (layer "F.Cu") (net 1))
 (segment (start 103.76625 95.27) (end 103.68875 95.1925) (width 0.2) (layer "F.Cu") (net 1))
 (segment (start 114.541984 94.47) (end 114.72875 94.47) (width 0.2) (layer "F.Cu") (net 1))
 (segment (start 106.17375 93.27) (end 105.81625 93.27) (width 0.2) (layer "F.Cu") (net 1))
 (segment (start 106.17375 92.4775) (end 104.48875 90.7925) (width 0.2) (layer "F.Cu") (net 1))
 (segment (start 110.60875 90.74) (end 110.62875 90.72) (width 0.2) (layer "F.Cu") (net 1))
 (segment (start 113.741984 95.27) (end 114.541984 94.47) (width 0.2) (layer "F.Cu") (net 1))
 (segment (start 104.21125 95.67) (end 103.68875 96.1925) (width 0.2) (layer "F.Cu") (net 7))
 (segment (start 106.17375 95.67) (end 104.21125 95.67) (width 0.2) (layer "F.Cu") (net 7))
 (segment (start 113.90875 94.537548) (end 113.90875 93.6925) (width 0.2) (layer "F.Cu") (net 7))
 (segment (start 106.17375 93.67) (end 105.06625 93.67) (width 0.2) (layer "F.Cu") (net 7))
 (segment (start 105.06625 93.67) (end 104.48875 93.0925) (width 0.2) (layer "F.Cu") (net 7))
 (segment (start 114.23125 93.37) (end 114.72875 93.37) (width 0.2) (layer "F.Cu") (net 7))
 (segment (start 113.576298 94.87) (end 113.90875 94.537548) (width 0.2) (layer "F.Cu") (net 7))
 (segment (start 113.90875 93.6925) (end 114.23125 93.37) (width 0.2) (layer "F.Cu") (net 7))
 (segment (start 113.04375 94.87) (end 113.576298 94.87) (width 0.2) (layer "F.Cu") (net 7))
 (segment (start 118.92875 97.26) (end 118.50875 97.68) (width 0.3) (layer "F.Cu") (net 4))
 (segment (start 118.92875 96.08) (end 118.92875 97.26) (width 0.3) (layer "F.Cu") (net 4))
 (segment (start 117.64875 93.56) (end 117.32875 93.88) (width 0.3) (layer "F.Cu") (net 5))
 (segment (start 117.64875 92.28) (end 117.64875 93.56) (width 0.3) (layer "F.Cu") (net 5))
 (segment (start 117.12875 93.68) (end 117.32875 93.88) (width 0.2) (layer "F.Cu") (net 5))
 (segment (start 114.59875 95.67) (end 114.69875 95.57) (width 0.2) (layer "F.Cu") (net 6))
 (segment (start 113.04375 95.67) (end 114.59875 95.67) (width 0.2) (layer "F.Cu") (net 6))
 (segment (start 102.40875 93.1925) (end 101.31875 93.1925) (width 0.2) (layer "F.Cu") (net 43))
 (segment (start 103.28625 94.07) (end 102.40875 93.1925) (width 0.2) (layer "F.Cu") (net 43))
 (segment (start 106.17375 94.07) (end 103.28625 94.07) (width 0.2) (layer "F.Cu") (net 43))
 (segment (start 101.39625 94.47) (end 101.31875 94.3925) (width 0.2) (layer "F.Cu") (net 9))
 (segment (start 106.17375 94.47) (end 101.39625 94.47) (width 0.2) (layer "F.Cu") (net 9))
 (segment (start 106.17375 98.07) (end 106.17375 99.52625) (width 0.2) (layer "F.Cu") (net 49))
 (segment (start 106.17375 99.52625) (end 106 99.7) (width 0.2) (layer "F.Cu") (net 49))
 (segment (start 106.17375 98.07) (end 105.995491 98.07) (width 0.2) (layer "F.Cu") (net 49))
 (via (at 106 99.7) (size 0.8) (drill 0.4) (layers "F.Cu" "B.Cu") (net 49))
 (segment (start 120.44 98.766396) (end 120.44 98.6) (width 0.2) (layer "B.Cu") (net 49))
 (segment (start 106 99.7) (end 106.8 100.5) (width 0.2) (layer "B.Cu") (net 49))
 (segment (start 118.706396 100.5) (end 120.44 98.766396) (width 0.2) (layer "B.Cu") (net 49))
 (segment (start 106.8 100.5) (end 118.706396 100.5) (width 0.2) (layer "B.Cu") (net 49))
 (segment (start 104.743504 96.07) (end 103.713504 97.1) (width 0.2) (layer "F.Cu") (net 44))
 (segment (start 103.713504 97.1) (end 103.2 97.1) (width 0.2) (layer "F.Cu") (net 44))
 (segment (start 104.743504 96.07) (end 106.17375 96.07) (width 0.2) (layer "F.Cu") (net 44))
 (via (at 103.2 97.1) (size 0.8) (drill 0.4) (layers "F.Cu" "B.Cu") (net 44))
 (segment (start 113.9 92.97) (end 113.9 91.634315) (width 0.2) (layer "B.Cu") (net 44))
 (segment (start 103.2 97.1) (end 109.77 97.1) (width 0.2) (layer "B.Cu") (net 44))
 (segment (start 118.2 89.9) (end 119.17 90.87) (width 0.2) (layer "B.Cu") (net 44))
 (segment (start 113.9 91.634315) (end 115.634315 89.9) (width 0.2) (layer "B.Cu") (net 44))
 (segment (start 119.17 90.87) (end 119.17 91.4) (width 0.2) (layer "B.Cu") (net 44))
 (segment (start 109.77 97.1) (end 113.9 92.97) (width 0.2) (layer "B.Cu") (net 44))
 (segment (start 115.634315 89.9) (end 118.2 89.9) (width 0.2) (layer "B.Cu") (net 44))
 (segment (start 103.57919 97.8) (end 102.5 97.8) (width 0.2) (layer "F.Cu") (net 45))
 (segment (start 106.17375 96.47) (end 104.90919 96.47) (width 0.2) (layer "F.Cu") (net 45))
 (segment (start 104.90919 96.47) (end 103.57919 97.8) (width 0.2) (layer "F.Cu") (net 45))
 (via (at 102.5 97.8) (size 0.8) (drill 0.4) (layers "F.Cu" "B.Cu") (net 45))
 (segment (start 117.9 90.8) (end 117.9 91.4) (width 0.2) (layer "B.Cu") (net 45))
 (segment (start 115.3 90.8) (end 114.3 91.8) (width 0.2) (layer "B.Cu") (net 45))
 (segment (start 115.3 90.8) (end 115.8 90.3) (width 0.2) (layer "B.Cu") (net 45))
 (segment (start 115.8 90.3) (end 117.4 90.3) (width 0.2) (layer "B.Cu") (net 45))
 (segment (start 102.5 97.8) (end 109.635686 97.8) (width 0.2) (layer "B.Cu") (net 45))
 (segment (start 117.4 90.3) (end 117.9 90.8) (width 0.2) (layer "B.Cu") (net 45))
 (segment (start 114.3 93.135686) (end 109.635686 97.8) (width 0.2) (layer "B.Cu") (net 45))
 (segment (start 114.3 92.8) (end 114.3 93.135686) (width 0.2) (layer "B.Cu") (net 45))
 (segment (start 114.3 91.8) (end 114.3 92.8) (width 0.2) (layer "B.Cu") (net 45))
 (segment (start 105.074876 96.87) (end 103.444876 98.5) (width 0.2) (layer "F.Cu") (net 46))
 (segment (start 106.17375 96.87) (end 105.074876 96.87) (width 0.2) (layer "F.Cu") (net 46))
 (segment (start 103.444876 98.5) (end 103.2 98.5) (width 0.2) (layer "F.Cu") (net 46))
 (via (at 103.2 98.5) (size 0.8) (drill 0.4) (layers "F.Cu" "B.Cu") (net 46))
 (segment (start 103.2 98.5) (end 103.5 98.2) (width 0.2) (layer "B.Cu") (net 46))
 (segment (start 103.5 98.2) (end 109.83 98.2) (width 0.2) (layer "B.Cu") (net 46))
 (segment (start 109.83 98.2) (end 116.63 91.4) (width 0.2) (layer "B.Cu") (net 46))
 (segment (start 116.555 91.576396) (end 116.555 91.41) (width 0.2) (layer "B.Cu") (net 46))
 (segment (start 116.63 91.4) (end 116.601371 91.4) (width 0.2) (layer "B.Cu") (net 46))
 (segment (start 106.17375 97.27) (end 105.240562 97.27) (width 0.2) (layer "F.Cu") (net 47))
 (segment (start 105.240562 97.27) (end 104.2 98.310562) (width 0.2) (layer "F.Cu") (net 47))
 (segment (start 104.2 98.310562) (end 104.2 98.9) (width 0.2) (layer "F.Cu") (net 47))
 (via (at 104.2 98.9) (size 0.8) (drill 0.4) (layers "F.Cu" "B.Cu") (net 47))
 (segment (start 117.9 98.9) (end 117.9 98.6) (width 0.2) (layer "B.Cu") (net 47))
 (segment (start 107.8 99.7) (end 116.966396 99.7) (width 0.2) (layer "B.Cu") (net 47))
 (segment (start 104.5 98.6) (end 106.7 98.6) (width 0.2) (layer "B.Cu") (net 47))
 (segment (start 117.9 98.766396) (end 117.9 98.6) (width 0.2) (layer "B.Cu") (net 47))
 (segment (start 116.966396 99.7) (end 117.9 98.766396) (width 0.2) (layer "B.Cu") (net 47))
 (segment (start 106.7 98.6) (end 107.8 99.7) (width 0.2) (layer "B.Cu") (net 47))
 (segment (start 104.2 98.9) (end 104.5 98.6) (width 0.2) (layer "B.Cu") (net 47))
 (segment (start 105.1 98.07) (end 105.1 99.3) (width 0.2) (layer "F.Cu") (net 48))
 (segment (start 105.5 97.67) (end 105.1 98.07) (width 0.2) (layer "F.Cu") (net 48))
 (segment (start 106.17375 97.67) (end 105.5 97.67) (width 0.2) (layer "F.Cu") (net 48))
 (via (at 105.1 99.3) (size 0.8) (drill 0.4) (layers "F.Cu" "B.Cu") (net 48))
 (segment (start 105.4 99) (end 106.5 99) (width 0.2) (layer "B.Cu") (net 48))
 (segment (start 107.6 100.1) (end 117.836396 100.1) (width 0.2) (layer "B.Cu") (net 48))
 (segment (start 117.836396 100.1) (end 119.17 98.766396) (width 0.2) (layer "B.Cu") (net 48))
 (segment (start 119.17 98.766396) (end 119.17 98.6) (width 0.2) (layer "B.Cu") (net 48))
 (segment (start 106.5 99) (end 107.6 100.1) (width 0.2) (layer "B.Cu") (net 48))
 (segment (start 105.1 99.3) (end 105.4 99) (width 0.2) (layer "B.Cu") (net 48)))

